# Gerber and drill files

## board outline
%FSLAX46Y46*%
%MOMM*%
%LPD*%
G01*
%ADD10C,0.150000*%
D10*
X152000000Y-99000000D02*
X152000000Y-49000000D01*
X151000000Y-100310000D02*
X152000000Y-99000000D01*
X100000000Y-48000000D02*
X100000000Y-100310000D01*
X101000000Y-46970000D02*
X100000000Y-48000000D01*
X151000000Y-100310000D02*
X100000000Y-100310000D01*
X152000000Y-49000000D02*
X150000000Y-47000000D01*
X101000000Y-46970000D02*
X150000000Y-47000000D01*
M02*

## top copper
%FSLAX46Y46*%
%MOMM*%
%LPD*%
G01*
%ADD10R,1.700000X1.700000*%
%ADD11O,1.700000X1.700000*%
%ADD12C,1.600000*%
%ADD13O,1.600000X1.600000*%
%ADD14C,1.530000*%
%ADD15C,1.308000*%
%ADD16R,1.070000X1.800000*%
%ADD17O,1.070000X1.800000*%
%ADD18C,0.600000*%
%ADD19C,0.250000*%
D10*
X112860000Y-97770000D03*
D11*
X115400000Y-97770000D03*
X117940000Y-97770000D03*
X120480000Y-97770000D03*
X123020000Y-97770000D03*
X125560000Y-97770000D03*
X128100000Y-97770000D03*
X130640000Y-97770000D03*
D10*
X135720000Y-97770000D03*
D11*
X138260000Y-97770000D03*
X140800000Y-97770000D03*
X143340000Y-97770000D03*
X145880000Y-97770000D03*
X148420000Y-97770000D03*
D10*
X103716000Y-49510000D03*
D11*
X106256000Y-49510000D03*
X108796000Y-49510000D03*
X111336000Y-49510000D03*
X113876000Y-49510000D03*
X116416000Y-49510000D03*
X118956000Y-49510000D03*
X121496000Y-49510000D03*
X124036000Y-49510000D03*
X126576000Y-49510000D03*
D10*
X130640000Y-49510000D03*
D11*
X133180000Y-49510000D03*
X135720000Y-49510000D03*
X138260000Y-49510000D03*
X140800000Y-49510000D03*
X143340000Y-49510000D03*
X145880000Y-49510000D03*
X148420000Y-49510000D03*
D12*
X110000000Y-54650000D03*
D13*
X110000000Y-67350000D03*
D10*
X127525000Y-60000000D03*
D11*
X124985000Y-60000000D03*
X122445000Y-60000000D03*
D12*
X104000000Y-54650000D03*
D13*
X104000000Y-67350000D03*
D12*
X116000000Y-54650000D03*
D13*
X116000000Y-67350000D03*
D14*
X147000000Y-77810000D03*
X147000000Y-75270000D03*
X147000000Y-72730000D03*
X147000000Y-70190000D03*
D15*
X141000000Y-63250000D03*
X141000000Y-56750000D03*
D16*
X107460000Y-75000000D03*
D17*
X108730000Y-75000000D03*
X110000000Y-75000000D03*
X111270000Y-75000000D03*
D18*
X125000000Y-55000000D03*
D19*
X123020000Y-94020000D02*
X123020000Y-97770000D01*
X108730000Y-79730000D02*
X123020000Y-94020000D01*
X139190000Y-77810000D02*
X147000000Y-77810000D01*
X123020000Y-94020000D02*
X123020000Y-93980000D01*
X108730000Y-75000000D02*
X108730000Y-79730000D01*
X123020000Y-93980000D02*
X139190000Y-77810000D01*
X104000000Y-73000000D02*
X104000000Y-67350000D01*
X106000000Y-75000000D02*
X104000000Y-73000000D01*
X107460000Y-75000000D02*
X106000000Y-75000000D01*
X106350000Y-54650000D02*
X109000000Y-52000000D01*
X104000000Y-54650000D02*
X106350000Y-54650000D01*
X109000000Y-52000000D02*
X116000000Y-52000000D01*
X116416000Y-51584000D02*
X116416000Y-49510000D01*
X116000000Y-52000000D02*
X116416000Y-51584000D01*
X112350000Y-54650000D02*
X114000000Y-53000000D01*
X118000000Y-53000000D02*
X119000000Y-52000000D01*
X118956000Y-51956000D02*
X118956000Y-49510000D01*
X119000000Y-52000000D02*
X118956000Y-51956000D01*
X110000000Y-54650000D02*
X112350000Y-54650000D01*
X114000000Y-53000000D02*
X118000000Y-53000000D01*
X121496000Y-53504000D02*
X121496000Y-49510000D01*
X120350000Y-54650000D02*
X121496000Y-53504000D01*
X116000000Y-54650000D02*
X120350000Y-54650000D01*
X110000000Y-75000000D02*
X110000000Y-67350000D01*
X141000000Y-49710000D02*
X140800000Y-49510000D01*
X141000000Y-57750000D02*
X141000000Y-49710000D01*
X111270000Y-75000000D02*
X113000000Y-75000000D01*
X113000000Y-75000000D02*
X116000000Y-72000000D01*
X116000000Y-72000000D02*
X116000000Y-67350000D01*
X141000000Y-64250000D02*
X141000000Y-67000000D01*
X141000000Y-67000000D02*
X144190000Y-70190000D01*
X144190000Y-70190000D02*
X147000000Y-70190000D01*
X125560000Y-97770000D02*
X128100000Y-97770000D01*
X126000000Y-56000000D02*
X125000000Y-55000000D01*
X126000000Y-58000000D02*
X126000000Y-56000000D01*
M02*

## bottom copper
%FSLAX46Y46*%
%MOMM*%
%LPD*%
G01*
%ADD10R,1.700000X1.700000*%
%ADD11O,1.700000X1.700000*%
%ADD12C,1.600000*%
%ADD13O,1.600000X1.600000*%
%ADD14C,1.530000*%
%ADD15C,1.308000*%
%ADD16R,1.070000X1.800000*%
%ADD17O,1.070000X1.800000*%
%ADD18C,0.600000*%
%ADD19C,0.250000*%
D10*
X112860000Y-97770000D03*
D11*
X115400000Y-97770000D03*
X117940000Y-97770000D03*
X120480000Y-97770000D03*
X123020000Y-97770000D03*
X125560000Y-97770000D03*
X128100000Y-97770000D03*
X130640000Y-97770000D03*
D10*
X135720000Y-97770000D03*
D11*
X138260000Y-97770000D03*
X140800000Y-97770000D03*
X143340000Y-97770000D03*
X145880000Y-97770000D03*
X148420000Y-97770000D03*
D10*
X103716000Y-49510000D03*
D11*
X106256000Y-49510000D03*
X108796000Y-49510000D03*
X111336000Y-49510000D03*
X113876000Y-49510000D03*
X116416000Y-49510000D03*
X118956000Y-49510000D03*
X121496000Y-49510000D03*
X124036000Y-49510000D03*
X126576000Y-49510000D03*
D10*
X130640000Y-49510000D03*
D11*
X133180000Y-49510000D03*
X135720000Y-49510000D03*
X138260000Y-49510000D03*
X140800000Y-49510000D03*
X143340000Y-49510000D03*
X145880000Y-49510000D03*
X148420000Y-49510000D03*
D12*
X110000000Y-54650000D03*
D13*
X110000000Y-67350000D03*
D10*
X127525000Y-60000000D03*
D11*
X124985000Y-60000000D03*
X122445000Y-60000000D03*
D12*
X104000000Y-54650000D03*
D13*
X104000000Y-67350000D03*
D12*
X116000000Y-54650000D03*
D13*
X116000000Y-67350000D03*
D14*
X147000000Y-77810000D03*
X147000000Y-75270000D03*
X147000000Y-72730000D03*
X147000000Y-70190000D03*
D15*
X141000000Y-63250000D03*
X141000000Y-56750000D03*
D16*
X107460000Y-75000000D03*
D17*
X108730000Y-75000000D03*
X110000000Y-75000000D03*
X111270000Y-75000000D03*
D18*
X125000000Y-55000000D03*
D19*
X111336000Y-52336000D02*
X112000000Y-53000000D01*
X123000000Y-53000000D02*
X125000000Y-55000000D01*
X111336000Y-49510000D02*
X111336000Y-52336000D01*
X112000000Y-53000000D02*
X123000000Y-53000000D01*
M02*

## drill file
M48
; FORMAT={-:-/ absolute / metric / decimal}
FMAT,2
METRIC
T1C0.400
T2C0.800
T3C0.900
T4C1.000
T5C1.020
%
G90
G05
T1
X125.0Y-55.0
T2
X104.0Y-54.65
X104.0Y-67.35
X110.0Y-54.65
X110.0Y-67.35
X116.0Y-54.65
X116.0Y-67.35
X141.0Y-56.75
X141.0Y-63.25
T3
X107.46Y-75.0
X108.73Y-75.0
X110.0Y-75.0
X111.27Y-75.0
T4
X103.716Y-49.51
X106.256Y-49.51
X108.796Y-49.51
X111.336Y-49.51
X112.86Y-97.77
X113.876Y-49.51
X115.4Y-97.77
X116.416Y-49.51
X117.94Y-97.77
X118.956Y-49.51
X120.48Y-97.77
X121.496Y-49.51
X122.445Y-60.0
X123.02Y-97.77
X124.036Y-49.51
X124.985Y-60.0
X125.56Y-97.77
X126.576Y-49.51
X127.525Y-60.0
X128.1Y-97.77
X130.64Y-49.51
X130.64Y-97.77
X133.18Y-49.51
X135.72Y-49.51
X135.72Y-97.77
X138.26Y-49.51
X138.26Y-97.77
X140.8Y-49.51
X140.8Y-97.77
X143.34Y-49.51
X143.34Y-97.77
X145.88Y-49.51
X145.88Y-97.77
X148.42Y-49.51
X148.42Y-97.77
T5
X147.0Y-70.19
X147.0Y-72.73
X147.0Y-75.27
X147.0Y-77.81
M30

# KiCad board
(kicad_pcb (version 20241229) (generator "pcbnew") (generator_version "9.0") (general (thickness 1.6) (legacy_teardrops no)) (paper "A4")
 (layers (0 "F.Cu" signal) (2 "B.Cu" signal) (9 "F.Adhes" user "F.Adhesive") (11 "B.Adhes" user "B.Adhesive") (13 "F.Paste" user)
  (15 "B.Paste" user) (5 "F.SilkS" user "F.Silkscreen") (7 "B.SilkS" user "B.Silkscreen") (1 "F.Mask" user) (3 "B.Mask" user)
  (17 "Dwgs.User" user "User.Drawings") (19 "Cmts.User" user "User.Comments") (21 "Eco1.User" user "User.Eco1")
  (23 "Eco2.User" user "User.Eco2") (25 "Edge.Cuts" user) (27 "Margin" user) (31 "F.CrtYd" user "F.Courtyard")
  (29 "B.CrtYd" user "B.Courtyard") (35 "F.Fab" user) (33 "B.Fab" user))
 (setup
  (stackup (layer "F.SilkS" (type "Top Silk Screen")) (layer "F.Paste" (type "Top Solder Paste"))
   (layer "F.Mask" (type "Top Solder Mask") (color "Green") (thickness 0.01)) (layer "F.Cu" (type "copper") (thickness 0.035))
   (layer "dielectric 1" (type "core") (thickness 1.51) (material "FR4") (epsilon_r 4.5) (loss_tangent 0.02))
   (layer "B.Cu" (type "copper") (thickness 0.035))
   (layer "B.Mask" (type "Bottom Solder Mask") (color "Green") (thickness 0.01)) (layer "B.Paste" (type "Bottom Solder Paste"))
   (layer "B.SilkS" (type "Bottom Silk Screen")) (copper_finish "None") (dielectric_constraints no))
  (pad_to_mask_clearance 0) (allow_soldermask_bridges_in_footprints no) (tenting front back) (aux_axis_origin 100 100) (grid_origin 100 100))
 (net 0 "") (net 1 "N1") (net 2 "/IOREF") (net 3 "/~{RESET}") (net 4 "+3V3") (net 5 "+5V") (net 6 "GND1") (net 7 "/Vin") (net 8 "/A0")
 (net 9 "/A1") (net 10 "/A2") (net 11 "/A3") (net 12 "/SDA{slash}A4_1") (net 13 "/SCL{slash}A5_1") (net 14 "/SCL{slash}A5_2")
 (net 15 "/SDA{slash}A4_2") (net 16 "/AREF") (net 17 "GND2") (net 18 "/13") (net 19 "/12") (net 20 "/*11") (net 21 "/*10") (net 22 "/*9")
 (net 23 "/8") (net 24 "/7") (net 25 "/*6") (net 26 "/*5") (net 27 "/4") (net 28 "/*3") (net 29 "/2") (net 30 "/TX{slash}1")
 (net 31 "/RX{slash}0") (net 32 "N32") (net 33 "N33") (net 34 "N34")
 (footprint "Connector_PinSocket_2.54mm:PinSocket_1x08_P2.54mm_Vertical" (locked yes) (layer "F.Cu") (at 112.86 97.77 90)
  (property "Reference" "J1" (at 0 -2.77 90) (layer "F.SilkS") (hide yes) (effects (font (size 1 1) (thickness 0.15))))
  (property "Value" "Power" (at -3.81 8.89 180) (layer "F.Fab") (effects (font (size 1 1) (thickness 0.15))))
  (pad "1" thru_hole rect (at 0 0 90) (size 1.7 1.7) (drill 1) (layers "*.Cu" "*.Mask") (remove_unused_layers no) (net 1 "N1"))
  (pad "2" thru_hole oval (at 0 2.54 90) (size 1.7 1.7) (drill 1) (layers "*.Cu" "*.Mask") (remove_unused_layers no) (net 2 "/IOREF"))
  (pad "3" thru_hole oval (at 0 5.08 90) (size 1.7 1.7) (drill 1) (layers "*.Cu" "*.Mask") (remove_unused_layers no) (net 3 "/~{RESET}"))
  (pad "4" thru_hole oval (at 0 7.62 90) (size 1.7 1.7) (drill 1) (layers "*.Cu" "*.Mask") (remove_unused_layers no) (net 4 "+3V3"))
  (pad "5" thru_hole oval (at 0 10.16 90) (size 1.7 1.7) (drill 1) (layers "*.Cu" "*.Mask") (remove_unused_layers no) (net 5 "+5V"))
  (pad "6" thru_hole oval (at 0 12.7 90) (size 1.7 1.7) (drill 1) (layers "*.Cu" "*.Mask") (remove_unused_layers no) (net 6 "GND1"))
  (pad "7" thru_hole oval (at 0 15.24 90) (size 1.7 1.7) (drill 1) (layers "*.Cu" "*.Mask") (remove_unused_layers no) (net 6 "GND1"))
  (pad "8" thru_hole oval (at 0 17.78 90) (size 1.7 1.7) (drill 1) (layers "*.Cu" "*.Mask") (remove_unused_layers no) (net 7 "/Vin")))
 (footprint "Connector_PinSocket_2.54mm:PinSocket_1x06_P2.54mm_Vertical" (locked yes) (layer "F.Cu") (at 135.72 97.77 90)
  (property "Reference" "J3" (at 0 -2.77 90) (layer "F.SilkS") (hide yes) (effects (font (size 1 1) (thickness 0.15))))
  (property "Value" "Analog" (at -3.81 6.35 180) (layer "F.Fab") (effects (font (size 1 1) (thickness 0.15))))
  (pad "1" thru_hole rect (at 0 0 90) (size 1.7 1.7) (drill 1) (layers "*.Cu" "*.Mask") (remove_unused_layers no) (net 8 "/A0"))
  (pad "2" thru_hole oval (at 0 2.54 90) (size 1.7 1.7) (drill 1) (layers "*.Cu" "*.Mask") (remove_unused_layers no) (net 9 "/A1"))
  (pad "3" thru_hole oval (at 0 5.08 90) (size 1.7 1.7) (drill 1) (layers "*.Cu" "*.Mask") (remove_unused_layers no) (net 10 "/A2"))
  (pad "4" thru_hole oval (at 0 7.62 90) (size 1.7 1.7) (drill 1) (layers "*.Cu" "*.Mask") (remove_unused_layers no) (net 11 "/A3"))
  (pad "5" thru_hole oval (at 0 10.16 90) (size 1.7 1.7) (drill 1) (layers "*.Cu" "*.Mask") (remove_unused_layers no)
   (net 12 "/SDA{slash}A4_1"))
  (pad "6" thru_hole oval (at 0 12.7 90) (size 1.7 1.7) (drill 1) (layers "*.Cu" "*.Mask") (remove_unused_layers no)
   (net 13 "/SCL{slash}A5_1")))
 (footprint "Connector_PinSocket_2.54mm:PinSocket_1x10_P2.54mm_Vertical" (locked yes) (layer "F.Cu") (at 103.716 49.51 90)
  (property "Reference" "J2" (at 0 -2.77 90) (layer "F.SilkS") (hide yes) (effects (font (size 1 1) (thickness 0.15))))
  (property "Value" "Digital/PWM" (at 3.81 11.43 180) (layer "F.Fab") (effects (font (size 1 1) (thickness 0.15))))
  (pad "1" thru_hole rect (at 0 0 90) (size 1.7 1.7) (drill 1) (layers "*.Cu" "*.Mask") (remove_unused_layers no) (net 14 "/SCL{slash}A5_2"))
  (pad "2" thru_hole oval (at 0 2.54 90) (size 1.7 1.7) (drill 1) (layers "*.Cu" "*.Mask") (remove_unused_layers no)
   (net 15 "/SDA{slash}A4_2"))
  (pad "3" thru_hole oval (at 0 5.08 90) (size 1.7 1.7) (drill 1) (layers "*.Cu" "*.Mask") (remove_unused_layers no) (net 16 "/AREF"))
  (pad "4" thru_hole oval (at 0 7.62 90) (size 1.7 1.7) (drill 1) (layers "*.Cu" "*.Mask") (remove_unused_layers no) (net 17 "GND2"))
  (pad "5" thru_hole oval (at 0 10.16 90) (size 1.7 1.7) (drill 1) (layers "*.Cu" "*.Mask") (remove_unused_layers no) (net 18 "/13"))
  (pad "6" thru_hole oval (at 0 12.7 90) (size 1.7 1.7) (drill 1) (layers "*.Cu" "*.Mask") (remove_unused_layers no) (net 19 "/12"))
  (pad "7" thru_hole oval (at 0 15.24 90) (size 1.7 1.7) (drill 1) (layers "*.Cu" "*.Mask") (remove_unused_layers no) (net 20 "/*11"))
  (pad "8" thru_hole oval (at 0 17.78 90) (size 1.7 1.7) (drill 1) (layers "*.Cu" "*.Mask") (remove_unused_layers no) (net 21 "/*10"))
  (pad "9" thru_hole oval (at 0 20.32 90) (size 1.7 1.7) (drill 1) (layers "*.Cu" "*.Mask") (remove_unused_layers no) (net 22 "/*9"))
  (pad "10" thru_hole oval (at 0 22.86 90) (size 1.7 1.7) (drill 1) (layers "*.Cu" "*.Mask") (remove_unused_layers no) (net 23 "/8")))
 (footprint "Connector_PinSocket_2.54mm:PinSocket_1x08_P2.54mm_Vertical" (layer "F.Cu") (at 130.64 49.51 90)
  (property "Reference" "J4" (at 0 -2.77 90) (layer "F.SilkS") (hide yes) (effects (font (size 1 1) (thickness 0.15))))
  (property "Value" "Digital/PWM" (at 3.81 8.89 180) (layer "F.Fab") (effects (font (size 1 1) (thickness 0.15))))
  (pad "1" thru_hole rect (at 0 0 90) (size 1.7 1.7) (drill 1) (layers "*.Cu" "*.Mask") (remove_unused_layers no) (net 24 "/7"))
  (pad "2" thru_hole oval (at 0 2.54 90) (size 1.7 1.7) (drill 1) (layers "*.Cu" "*.Mask") (remove_unused_layers no) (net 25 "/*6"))
  (pad "3" thru_hole oval (at 0 5.08 90) (size 1.7 1.7) (drill 1) (layers "*.Cu" "*.Mask") (remove_unused_layers no) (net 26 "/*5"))
  (pad "4" thru_hole oval (at 0 7.62 90) (size 1.7 1.7) (drill 1) (layers "*.Cu" "*.Mask") (remove_unused_layers no) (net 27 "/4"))
  (pad "5" thru_hole oval (at 0 10.16 90) (size 1.7 1.7) (drill 1) (layers "*.Cu" "*.Mask") (remove_unused_layers no) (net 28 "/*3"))
  (pad "6" thru_hole oval (at 0 12.7 90) (size 1.7 1.7) (drill 1) (layers "*.Cu" "*.Mask") (remove_unused_layers no) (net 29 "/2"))
  (pad "7" thru_hole oval (at 0 15.24 90) (size 1.7 1.7) (drill 1) (layers "*.Cu" "*.Mask") (remove_unused_layers no) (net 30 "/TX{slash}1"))
  (pad "8" thru_hole oval (at 0 17.78 90) (size 1.7 1.7) (drill 1) (layers "*.Cu" "*.Mask") (remove_unused_layers no) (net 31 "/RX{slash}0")))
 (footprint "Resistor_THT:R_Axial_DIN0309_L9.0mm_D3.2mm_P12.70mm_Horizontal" (layer "F.Cu") (at 110 54.65 -90)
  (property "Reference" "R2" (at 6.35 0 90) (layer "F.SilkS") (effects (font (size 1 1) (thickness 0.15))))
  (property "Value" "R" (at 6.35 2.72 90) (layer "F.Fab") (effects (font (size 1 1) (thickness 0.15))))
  (pad "1" thru_hole circle (at 0 0 270) (size 1.6 1.6) (drill 0.8) (layers "*.Cu" "*.Mask") (remove_unused_layers no) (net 20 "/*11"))
  (pad "2" thru_hole oval (at 12.7 0 270) (size 1.6 1.6) (drill 0.8) (layers "*.Cu" "*.Mask") (remove_unused_layers no) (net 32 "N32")))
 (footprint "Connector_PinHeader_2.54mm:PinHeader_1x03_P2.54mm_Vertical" (layer "F.Cu") (at 127.525 60 -90)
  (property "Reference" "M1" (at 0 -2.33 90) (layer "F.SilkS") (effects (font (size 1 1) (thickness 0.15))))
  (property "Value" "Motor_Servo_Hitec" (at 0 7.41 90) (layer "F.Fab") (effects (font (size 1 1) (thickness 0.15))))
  (pad "1" thru_hole rect (at 0 0 270) (size 1.7 1.7) (drill 1) (layers "*.Cu" "*.Mask") (remove_unused_layers no) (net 22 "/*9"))
  (pad "2" thru_hole oval (at 0 2.54 270) (size 1.7 1.7) (drill 1) (layers "*.Cu" "*.Mask") (remove_unused_layers no) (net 5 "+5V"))
  (pad "3" thru_hole oval (at 0 5.08 270) (size 1.7 1.7) (drill 1) (layers "*.Cu" "*.Mask") (remove_unused_layers no) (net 17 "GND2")))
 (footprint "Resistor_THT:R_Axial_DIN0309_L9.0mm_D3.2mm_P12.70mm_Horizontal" (layer "F.Cu") (at 104 54.65 -90)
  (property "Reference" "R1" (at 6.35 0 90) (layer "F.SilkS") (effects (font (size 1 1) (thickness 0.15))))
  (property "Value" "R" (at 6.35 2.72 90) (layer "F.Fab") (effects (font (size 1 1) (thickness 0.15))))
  (pad "1" thru_hole circle (at 0 0 270) (size 1.6 1.6) (drill 0.8) (layers "*.Cu" "*.Mask") (remove_unused_layers no) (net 19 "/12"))
  (pad "2" thru_hole oval (at 12.7 0 270) (size 1.6 1.6) (drill 0.8) (layers "*.Cu" "*.Mask") (remove_unused_layers no) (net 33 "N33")))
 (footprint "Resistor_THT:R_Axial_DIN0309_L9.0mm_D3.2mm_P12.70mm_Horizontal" (layer "F.Cu") (at 116 54.65 -90)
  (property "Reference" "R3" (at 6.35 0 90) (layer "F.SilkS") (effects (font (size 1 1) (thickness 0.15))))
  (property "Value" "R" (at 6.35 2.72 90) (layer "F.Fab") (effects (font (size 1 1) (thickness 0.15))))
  (pad "1" thru_hole circle (at 0 0 270) (size 1.6 1.6) (drill 0.8) (layers "*.Cu" "*.Mask") (remove_unused_layers no) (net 21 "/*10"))
  (pad "2" thru_hole oval (at 12.7 0 270) (size 1.6 1.6) (drill 0.8) (layers "*.Cu" "*.Mask") (remove_unused_layers no) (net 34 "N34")))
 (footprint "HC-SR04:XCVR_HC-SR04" (layer "F.Cu") (at 147 74 90)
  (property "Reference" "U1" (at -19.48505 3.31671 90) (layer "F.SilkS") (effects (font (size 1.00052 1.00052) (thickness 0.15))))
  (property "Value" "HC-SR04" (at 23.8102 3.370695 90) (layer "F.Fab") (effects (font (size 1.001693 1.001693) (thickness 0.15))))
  (pad "1" thru_hole circle (at -3.81 0 90) (size 1.53 1.53) (drill 1.02) (layers "*.Cu" "*.Mask") (remove_unused_layers no) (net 5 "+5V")
   (solder_mask_margin 0.102))
  (pad "2" thru_hole circle (at -1.27 0 90) (size 1.53 1.53) (drill 1.02) (layers "*.Cu" "*.Mask") (remove_unused_layers no) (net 26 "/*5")
   (solder_mask_margin 0.102))
  (pad "3" thru_hole circle (at 1.27 0 90) (size 1.53 1.53) (drill 1.02) (layers "*.Cu" "*.Mask") (remove_unused_layers no) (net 25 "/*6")
   (solder_mask_margin 0.102))
  (pad "4" thru_hole circle (at 3.81 0 90) (size 1.53 1.53) (drill 1.02) (layers "*.Cu" "*.Mask") (remove_unused_layers no) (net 6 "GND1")
   (solder_mask_margin 0.102)))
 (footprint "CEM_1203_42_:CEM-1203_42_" (layer "F.Cu") (at 141 60 -90)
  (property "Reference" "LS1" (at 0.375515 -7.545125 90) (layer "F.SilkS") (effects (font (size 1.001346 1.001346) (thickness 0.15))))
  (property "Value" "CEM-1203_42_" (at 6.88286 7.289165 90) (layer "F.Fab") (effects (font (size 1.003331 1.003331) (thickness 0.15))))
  (pad "N" thru_hole circle (at 3.25 0 270) (size 1.308 1.308) (drill 0.8) (layers "*.Cu" "*.Mask") (remove_unused_layers no) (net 6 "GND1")
   (solder_mask_margin 0.102))
  (pad "P" thru_hole circle (at -3.25 0 270) (size 1.308 1.308) (drill 0.8) (layers "*.Cu" "*.Mask") (remove_unused_layers no)
   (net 28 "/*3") (solder_mask_margin 0.102)))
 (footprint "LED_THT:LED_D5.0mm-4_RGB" (layer "F.Cu") (at 107.46 75)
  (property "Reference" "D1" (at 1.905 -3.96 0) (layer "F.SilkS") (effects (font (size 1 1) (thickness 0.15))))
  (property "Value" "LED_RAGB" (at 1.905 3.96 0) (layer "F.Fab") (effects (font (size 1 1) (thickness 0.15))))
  (pad "1" thru_hole rect (at 0 0) (size 1.07 1.8) (drill 0.9) (layers "*.Cu" "*.Mask") (remove_unused_layers no) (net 33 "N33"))
  (pad "2" thru_hole oval (at 1.27 0) (size 1.07 1.8) (drill 0.9) (layers "*.Cu" "*.Mask") (remove_unused_layers no) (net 5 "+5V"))
  (pad "3" thru_hole oval (at 2.54 0) (size 1.07 1.8) (drill 0.9) (layers "*.Cu" "*.Mask") (remove_unused_layers no) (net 32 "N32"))
  (pad "4" thru_hole oval (at 3.81 0) (size 1.07 1.8) (drill 0.9) (layers "*.Cu" "*.Mask") (remove_unused_layers no) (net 34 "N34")))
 (gr_line (start 152 99) (end 152 49) (stroke (width 0.15) (type default)) (layer "Edge.Cuts"))
 (gr_line (start 151 100.31) (end 152 99) (stroke (width 0.15) (type default)) (layer "Edge.Cuts"))
 (gr_line (start 100 48) (end 100 100.31) (stroke (width 0.15) (type default)) (layer "Edge.Cuts"))
 (gr_line (start 101 46.97) (end 100 48) (stroke (width 0.15) (type default)) (layer "Edge.Cuts"))
 (gr_line (start 151 100.31) (end 100 100.31) (stroke (width 0.15) (type solid)) (layer "Edge.Cuts"))
 (gr_line (start 152 49) (end 150 47) (stroke (width 0.15) (type default)) (layer "Edge.Cuts"))
 (gr_line (start 101 46.97) (end 150 47) (stroke (width 0.15) (type solid)) (layer "Edge.Cuts"))
 (segment (start 123.02 94.02) (end 123.02 97.77) (width 0.25) (layer "F.Cu") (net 5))
 (segment (start 108.73 79.73) (end 123.02 94.02) (width 0.25) (layer "F.Cu") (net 5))
 (segment (start 139.19 77.81) (end 147 77.81) (width 0.25) (layer "F.Cu") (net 5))
 (segment (start 123.02 94.02) (end 123.02 93.98) (width 0.25) (layer "F.Cu") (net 5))
 (segment (start 108.73 75) (end 108.73 79.73) (width 0.25) (layer "F.Cu") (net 5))
 (segment (start 123.02 93.98) (end 139.19 77.81) (width 0.25) (layer "F.Cu") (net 5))
 (segment (start 104 73) (end 104 67.35) (width 0.25) (layer "F.Cu") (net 33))
 (segment (start 106 75) (end 104 73) (width 0.25) (layer "F.Cu") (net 33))
 (segment (start 107.46 75) (end 106 75) (width 0.25) (layer "F.Cu") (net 33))
 (segment (start 106.35 54.65) (end 109 52) (width 0.25) (layer "F.Cu") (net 19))
 (segment (start 104 54.65) (end 106.35 54.65) (width 0.25) (layer "F.Cu") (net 19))
 (segment (start 109 52) (end 116 52) (width 0.25) (layer "F.Cu") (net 19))
 (segment (start 116.416 51.584) (end 116.416 49.51) (width 0.25) (layer "F.Cu") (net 19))
 (segment (start 116 52) (end 116.416 51.584) (width 0.25) (layer "F.Cu") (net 19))
 (segment (start 112.35 54.65) (end 114 53) (width 0.25) (layer "F.Cu") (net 20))
 (segment (start 118 53) (end 119 52) (width 0.25) (layer "F.Cu") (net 20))
 (segment (start 118.956 51.956) (end 118.956 49.51) (width 0.25) (layer "F.Cu") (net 20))
 (segment (start 119 52) (end 118.956 51.956) (width 0.25) (layer "F.Cu") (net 20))
 (segment (start 110 54.65) (end 112.35 54.65) (width 0.25) (layer "F.Cu") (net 20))
 (segment (start 114 53) (end 118 53) (width 0.25) (layer "F.Cu") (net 20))
 (segment (start 121.496 53.504) (end 121.496 49.51) (width 0.25) (layer "F.Cu") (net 21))
 (segment (start 120.35 54.65) (end 121.496 53.504) (width 0.25) (layer "F.Cu") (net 21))
 (segment (start 116 54.65) (end 120.35 54.65) (width 0.25) (layer "F.Cu") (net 21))
 (segment (start 110 75) (end 110 67.35) (width 0.25) (layer "F.Cu") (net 32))
 (segment (start 141 49.71) (end 140.8 49.51) (width 0.25) (layer "F.Cu") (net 28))
 (segment (start 141 57.75) (end 141 49.71) (width 0.25) (layer "F.Cu") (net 28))
 (segment (start 111.27 75) (end 113 75) (width 0.25) (layer "F.Cu") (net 34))
 (segment (start 113 75) (end 116 72) (width 0.25) (layer "F.Cu") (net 34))
 (segment (start 116 72) (end 116 67.35) (width 0.25) (layer "F.Cu") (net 34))
 (segment (start 141 64.25) (end 141 67) (width 0.25) (layer "F.Cu") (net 6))
 (segment (start 141 67) (end 144.19 70.19) (width 0.25) (layer "F.Cu") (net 6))
 (segment (start 144.19 70.19) (end 147 70.19) (width 0.25) (layer "F.Cu") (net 6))
 (segment (start 125.56 97.77) (end 128.1 97.77) (width 0.25) (layer "F.Cu") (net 6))
 (segment (start 126 56) (end 125 55) (width 0.25) (layer "F.Cu") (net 17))
 (segment (start 126 58) (end 126 56) (width 0.25) (layer "F.Cu") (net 17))
 (via (at 125 55) (size 0.6) (drill 0.4) (layers "F.Cu" "B.Cu") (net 17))
 (segment (start 111.336 52.336) (end 112 53) (width 0.25) (layer "B.Cu") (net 17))
 (segment (start 123 53) (end 125 55) (width 0.25) (layer "B.Cu") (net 17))
 (segment (start 111.336 49.51) (end 111.336 52.336) (width 0.25) (layer "B.Cu") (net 17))
 (segment (start 112 53) (end 123 53) (width 0.25) (layer "B.Cu") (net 17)))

